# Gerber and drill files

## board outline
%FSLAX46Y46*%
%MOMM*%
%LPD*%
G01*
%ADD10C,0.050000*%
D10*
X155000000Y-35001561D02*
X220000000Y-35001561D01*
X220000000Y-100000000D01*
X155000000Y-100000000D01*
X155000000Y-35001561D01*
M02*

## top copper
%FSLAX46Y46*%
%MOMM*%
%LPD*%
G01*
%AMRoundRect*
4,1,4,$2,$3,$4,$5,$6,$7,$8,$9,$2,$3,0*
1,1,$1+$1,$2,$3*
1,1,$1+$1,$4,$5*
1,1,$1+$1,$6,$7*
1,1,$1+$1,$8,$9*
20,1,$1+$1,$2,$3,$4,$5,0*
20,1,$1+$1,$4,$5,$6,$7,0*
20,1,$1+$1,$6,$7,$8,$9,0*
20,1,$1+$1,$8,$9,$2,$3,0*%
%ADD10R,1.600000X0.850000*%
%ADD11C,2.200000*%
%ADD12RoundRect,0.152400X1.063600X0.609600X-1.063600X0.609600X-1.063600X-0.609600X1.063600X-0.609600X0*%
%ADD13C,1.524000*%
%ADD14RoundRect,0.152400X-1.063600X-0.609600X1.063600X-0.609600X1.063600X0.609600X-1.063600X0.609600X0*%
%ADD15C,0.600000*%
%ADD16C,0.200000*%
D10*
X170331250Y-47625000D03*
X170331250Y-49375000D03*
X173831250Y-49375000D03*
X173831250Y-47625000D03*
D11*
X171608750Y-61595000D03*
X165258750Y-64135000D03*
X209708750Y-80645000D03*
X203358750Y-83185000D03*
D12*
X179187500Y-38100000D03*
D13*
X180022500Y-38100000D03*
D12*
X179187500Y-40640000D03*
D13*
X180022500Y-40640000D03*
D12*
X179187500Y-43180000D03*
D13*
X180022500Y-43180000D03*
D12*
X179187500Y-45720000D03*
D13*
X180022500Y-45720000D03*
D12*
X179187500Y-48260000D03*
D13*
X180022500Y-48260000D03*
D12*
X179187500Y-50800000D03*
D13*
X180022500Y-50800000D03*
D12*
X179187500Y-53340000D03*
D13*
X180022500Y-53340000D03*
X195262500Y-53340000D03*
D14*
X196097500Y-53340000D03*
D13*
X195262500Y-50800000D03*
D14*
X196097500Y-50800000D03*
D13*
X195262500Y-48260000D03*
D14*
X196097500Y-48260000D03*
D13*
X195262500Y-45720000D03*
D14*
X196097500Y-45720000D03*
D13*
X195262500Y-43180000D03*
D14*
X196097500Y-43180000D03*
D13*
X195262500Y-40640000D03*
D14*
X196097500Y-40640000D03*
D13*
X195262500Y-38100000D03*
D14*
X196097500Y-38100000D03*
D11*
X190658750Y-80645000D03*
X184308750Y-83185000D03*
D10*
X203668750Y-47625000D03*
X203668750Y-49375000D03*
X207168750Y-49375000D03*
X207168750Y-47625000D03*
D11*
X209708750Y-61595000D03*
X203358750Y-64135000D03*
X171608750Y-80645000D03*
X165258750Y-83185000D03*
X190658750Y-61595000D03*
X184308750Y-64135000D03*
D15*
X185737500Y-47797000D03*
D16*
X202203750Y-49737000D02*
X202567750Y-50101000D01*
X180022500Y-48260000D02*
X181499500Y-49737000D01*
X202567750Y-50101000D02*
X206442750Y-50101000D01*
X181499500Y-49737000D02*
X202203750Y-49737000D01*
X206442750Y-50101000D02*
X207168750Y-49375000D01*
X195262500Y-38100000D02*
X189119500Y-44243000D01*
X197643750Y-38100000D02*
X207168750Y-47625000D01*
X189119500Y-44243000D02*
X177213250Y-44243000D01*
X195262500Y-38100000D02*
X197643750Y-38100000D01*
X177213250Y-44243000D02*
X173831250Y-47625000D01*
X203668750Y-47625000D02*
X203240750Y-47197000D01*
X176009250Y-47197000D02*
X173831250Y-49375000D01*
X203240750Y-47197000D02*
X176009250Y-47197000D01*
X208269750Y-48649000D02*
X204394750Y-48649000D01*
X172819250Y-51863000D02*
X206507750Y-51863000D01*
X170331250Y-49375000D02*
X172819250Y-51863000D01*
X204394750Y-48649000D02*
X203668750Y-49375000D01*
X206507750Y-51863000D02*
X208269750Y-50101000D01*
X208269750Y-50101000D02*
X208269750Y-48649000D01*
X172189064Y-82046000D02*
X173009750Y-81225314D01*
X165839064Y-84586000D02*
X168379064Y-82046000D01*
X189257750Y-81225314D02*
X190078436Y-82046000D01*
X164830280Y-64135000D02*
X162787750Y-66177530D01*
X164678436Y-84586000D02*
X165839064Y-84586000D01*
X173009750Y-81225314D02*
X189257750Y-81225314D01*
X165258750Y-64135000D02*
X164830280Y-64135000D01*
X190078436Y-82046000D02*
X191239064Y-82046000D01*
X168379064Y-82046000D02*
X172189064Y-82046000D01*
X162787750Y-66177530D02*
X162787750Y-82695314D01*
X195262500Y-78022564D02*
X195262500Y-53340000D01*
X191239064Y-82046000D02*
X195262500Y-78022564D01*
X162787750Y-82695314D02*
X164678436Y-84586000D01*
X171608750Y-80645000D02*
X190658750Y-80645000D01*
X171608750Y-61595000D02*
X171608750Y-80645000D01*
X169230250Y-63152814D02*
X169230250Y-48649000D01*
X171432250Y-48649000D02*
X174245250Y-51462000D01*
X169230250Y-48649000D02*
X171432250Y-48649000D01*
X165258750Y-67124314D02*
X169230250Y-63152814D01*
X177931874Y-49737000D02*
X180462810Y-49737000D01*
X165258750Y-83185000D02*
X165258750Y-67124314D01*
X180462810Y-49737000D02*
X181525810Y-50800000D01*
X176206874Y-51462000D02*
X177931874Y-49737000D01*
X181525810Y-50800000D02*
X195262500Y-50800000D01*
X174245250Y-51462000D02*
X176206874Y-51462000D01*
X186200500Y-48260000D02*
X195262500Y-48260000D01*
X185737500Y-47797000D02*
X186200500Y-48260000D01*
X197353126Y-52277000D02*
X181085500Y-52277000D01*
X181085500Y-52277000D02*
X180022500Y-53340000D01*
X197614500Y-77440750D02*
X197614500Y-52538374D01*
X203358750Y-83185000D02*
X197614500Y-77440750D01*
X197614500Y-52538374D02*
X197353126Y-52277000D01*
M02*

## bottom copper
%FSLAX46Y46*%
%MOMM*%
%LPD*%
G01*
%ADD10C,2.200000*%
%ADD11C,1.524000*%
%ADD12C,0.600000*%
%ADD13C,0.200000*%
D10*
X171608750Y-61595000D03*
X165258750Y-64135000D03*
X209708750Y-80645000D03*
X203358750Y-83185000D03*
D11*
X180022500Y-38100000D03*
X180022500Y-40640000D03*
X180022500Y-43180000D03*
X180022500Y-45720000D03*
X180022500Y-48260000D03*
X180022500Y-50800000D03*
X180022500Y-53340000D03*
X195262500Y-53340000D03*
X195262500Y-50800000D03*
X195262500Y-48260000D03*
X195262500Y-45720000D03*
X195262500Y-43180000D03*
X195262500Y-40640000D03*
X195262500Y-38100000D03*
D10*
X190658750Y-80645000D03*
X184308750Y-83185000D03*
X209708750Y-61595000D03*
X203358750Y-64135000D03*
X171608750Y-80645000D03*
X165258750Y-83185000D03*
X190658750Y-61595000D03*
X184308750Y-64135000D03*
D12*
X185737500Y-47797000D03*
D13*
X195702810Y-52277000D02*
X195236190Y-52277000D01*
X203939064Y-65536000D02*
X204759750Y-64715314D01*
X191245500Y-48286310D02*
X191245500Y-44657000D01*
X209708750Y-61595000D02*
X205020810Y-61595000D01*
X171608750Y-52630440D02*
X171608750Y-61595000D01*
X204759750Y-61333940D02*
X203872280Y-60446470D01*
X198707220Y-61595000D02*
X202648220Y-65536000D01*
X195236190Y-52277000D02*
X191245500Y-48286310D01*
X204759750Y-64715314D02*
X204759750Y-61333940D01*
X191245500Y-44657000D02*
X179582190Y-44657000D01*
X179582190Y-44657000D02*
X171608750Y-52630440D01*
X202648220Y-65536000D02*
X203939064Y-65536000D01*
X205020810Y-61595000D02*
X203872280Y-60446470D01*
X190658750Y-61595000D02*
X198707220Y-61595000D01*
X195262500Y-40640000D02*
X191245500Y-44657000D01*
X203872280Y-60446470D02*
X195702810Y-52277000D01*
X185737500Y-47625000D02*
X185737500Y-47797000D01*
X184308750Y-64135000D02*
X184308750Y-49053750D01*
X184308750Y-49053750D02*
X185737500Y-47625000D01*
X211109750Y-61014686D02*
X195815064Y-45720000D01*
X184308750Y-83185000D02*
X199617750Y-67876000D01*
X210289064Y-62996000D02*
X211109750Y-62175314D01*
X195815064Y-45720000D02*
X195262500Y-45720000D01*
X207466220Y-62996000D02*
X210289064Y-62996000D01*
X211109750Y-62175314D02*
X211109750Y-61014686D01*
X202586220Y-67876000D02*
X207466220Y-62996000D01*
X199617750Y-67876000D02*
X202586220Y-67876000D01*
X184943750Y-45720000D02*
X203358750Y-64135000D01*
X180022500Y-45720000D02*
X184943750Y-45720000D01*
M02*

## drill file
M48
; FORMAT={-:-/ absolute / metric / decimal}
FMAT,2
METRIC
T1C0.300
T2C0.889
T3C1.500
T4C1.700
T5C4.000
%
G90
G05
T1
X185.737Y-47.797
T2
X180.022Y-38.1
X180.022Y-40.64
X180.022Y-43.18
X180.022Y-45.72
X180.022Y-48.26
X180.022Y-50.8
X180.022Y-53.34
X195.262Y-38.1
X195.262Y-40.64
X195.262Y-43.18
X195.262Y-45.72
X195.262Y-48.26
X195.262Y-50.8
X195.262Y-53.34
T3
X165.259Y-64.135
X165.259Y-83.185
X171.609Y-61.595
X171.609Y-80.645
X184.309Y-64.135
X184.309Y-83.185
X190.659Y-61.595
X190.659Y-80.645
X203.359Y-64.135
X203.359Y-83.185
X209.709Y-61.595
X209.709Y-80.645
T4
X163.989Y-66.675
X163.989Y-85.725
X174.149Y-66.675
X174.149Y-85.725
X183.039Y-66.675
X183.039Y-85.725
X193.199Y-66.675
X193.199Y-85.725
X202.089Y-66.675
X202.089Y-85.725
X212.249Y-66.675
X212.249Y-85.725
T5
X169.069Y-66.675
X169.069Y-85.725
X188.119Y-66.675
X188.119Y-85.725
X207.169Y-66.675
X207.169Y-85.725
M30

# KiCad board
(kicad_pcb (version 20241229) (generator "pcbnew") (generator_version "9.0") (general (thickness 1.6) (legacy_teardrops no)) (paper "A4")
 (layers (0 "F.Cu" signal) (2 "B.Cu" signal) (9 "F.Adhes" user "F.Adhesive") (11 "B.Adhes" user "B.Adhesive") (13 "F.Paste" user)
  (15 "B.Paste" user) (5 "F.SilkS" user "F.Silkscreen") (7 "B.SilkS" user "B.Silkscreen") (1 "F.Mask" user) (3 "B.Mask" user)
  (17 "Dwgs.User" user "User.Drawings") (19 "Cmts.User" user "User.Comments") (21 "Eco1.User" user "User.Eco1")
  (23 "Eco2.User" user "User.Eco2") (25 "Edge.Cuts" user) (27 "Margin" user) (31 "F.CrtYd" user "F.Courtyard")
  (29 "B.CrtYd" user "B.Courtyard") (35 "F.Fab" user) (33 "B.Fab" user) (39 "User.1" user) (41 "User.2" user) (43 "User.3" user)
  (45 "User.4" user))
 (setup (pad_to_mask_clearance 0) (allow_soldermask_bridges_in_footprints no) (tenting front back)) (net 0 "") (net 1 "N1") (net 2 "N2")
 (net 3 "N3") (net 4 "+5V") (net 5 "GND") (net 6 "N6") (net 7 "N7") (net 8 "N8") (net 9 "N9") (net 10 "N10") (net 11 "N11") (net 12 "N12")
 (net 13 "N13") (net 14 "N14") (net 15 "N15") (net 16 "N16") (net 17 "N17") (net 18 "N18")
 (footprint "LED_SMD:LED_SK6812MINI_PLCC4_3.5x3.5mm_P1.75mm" (layer "F.Cu") (at 172.08125 48.5)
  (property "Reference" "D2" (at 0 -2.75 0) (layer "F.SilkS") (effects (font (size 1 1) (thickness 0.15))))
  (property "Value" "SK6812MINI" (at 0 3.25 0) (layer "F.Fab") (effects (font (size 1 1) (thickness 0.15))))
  (pad "1" smd rect (at -1.75 -0.875) (size 1.6 0.85) (layers "F.Cu" "F.Mask" "F.Paste") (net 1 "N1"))
  (pad "2" smd rect (at -1.75 0.875) (size 1.6 0.85) (layers "F.Cu" "F.Mask" "F.Paste") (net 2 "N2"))
  (pad "3" smd rect (at 1.75 0.875) (size 1.6 0.85) (layers "F.Cu" "F.Mask" "F.Paste") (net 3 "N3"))
  (pad "4" smd rect (at 1.75 -0.875) (size 1.6 0.85) (layers "F.Cu" "F.Mask" "F.Paste") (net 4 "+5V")))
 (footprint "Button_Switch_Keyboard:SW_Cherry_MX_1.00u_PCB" (layer "F.Cu") (at 171.60875 61.595)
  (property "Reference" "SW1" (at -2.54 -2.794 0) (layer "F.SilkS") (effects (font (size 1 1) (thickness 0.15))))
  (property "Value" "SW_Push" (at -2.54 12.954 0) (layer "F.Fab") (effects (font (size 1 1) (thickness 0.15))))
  (pad "" np_thru_hole circle (at -7.62 5.08) (size 1.7 1.7) (drill 1.7) (layers "*.Cu" "*.Mask"))
  (pad "" np_thru_hole circle (at -2.54 5.08) (size 4 4) (drill 4) (layers "*.Cu" "*.Mask"))
  (pad "" np_thru_hole circle (at 2.54 5.08) (size 1.7 1.7) (drill 1.7) (layers "*.Cu" "*.Mask"))
  (pad "1" thru_hole circle (at 0 0) (size 2.2 2.2) (drill 1.5) (layers "*.Cu" "*.Mask") (remove_unused_layers no) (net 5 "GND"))
  (pad "2" thru_hole circle (at -6.35 2.54) (size 2.2 2.2) (drill 1.5) (layers "*.Cu" "*.Mask") (remove_unused_layers no) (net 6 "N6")))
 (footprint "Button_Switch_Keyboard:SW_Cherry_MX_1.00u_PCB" (layer "F.Cu") (at 209.70875 80.645)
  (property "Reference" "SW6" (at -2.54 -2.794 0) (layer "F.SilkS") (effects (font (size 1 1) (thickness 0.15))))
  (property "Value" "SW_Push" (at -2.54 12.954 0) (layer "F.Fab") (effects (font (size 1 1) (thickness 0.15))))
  (pad "" np_thru_hole circle (at -7.62 5.08) (size 1.7 1.7) (drill 1.7) (layers "*.Cu" "*.Mask"))
  (pad "" np_thru_hole circle (at -2.54 5.08) (size 4 4) (drill 4) (layers "*.Cu" "*.Mask"))
  (pad "" np_thru_hole circle (at 2.54 5.08) (size 1.7 1.7) (drill 1.7) (layers "*.Cu" "*.Mask"))
  (pad "1" thru_hole circle (at 0 0) (size 2.2 2.2) (drill 1.5) (layers "*.Cu" "*.Mask") (remove_unused_layers no) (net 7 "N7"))
  (pad "2" thru_hole circle (at -6.35 2.54) (size 2.2 2.2) (drill 1.5) (layers "*.Cu" "*.Mask") (remove_unused_layers no) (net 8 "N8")))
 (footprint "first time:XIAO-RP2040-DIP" (layer "F.Cu") (at 187.6425 45.72)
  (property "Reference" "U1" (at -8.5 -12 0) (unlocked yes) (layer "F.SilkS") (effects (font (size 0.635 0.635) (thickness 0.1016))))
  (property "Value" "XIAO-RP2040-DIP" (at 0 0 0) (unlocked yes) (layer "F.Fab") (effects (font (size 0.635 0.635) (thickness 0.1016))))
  (pad "1" smd roundrect (at -8.455 -7.62 180) (size 2.432 1.524) (layers "F.Cu" "F.Mask") (roundrect_rratio 0.1) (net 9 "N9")
   (thermal_bridge_angle 45))
  (pad "1" thru_hole circle (at -7.62 -7.62 180) (size 1.524 1.524) (drill 0.889) (layers "*.Cu" "*.Mask") (remove_unused_layers no)
   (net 9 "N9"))
  (pad "2" smd roundrect (at -8.455 -5.08 180) (size 2.432 1.524) (layers "F.Cu" "F.Mask") (roundrect_rratio 0.1) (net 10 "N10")
   (thermal_bridge_angle 45))
  (pad "2" thru_hole circle (at -7.62 -5.08 180) (size 1.524 1.524) (drill 0.889) (layers "*.Cu" "*.Mask") (remove_unused_layers no)
   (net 10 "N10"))
  (pad "3" smd roundrect (at -8.455 -2.54 180) (size 2.432 1.524) (layers "F.Cu" "F.Mask") (roundrect_rratio 0.1) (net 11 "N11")
   (thermal_bridge_angle 45))
  (pad "3" thru_hole circle (at -7.62 -2.54 180) (size 1.524 1.524) (drill 0.889) (layers "*.Cu" "*.Mask") (remove_unused_layers no)
   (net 11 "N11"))
  (pad "4" smd roundrect (at -8.455 0 180) (size 2.432 1.524) (layers "F.Cu" "F.Mask") (roundrect_rratio 0.1) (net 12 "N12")
   (thermal_bridge_angle 45))
  (pad "4" thru_hole circle (at -7.62 0 180) (size 1.524 1.524) (drill 0.889) (layers "*.Cu" "*.Mask") (remove_unused_layers no)
   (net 12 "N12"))
  (pad "5" smd roundrect (at -8.455 2.54 180) (size 2.432 1.524) (layers "F.Cu" "F.Mask") (roundrect_rratio 0.1) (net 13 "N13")
   (thermal_bridge_angle 45))
  (pad "5" thru_hole circle (at -7.62 2.54 180) (size 1.524 1.524) (drill 0.889) (layers "*.Cu" "*.Mask") (remove_unused_layers no)
   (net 13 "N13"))
  (pad "6" smd roundrect (at -8.455 5.08 180) (size 2.432 1.524) (layers "F.Cu" "F.Mask") (roundrect_rratio 0.1) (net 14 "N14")
   (thermal_bridge_angle 45))
  (pad "6" thru_hole circle (at -7.62 5.08 180) (size 1.524 1.524) (drill 0.889) (layers "*.Cu" "*.Mask") (remove_unused_layers no)
   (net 14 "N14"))
  (pad "7" smd roundrect (at -8.455 7.62 180) (size 2.432 1.524) (layers "F.Cu" "F.Mask") (roundrect_rratio 0.1) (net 8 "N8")
   (thermal_bridge_angle 45))
  (pad "7" thru_hole circle (at -7.62 7.62 180) (size 1.524 1.524) (drill 0.889) (layers "*.Cu" "*.Mask") (remove_unused_layers no)
   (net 8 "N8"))
  (pad "8" thru_hole circle (at 7.62 7.62) (size 1.524 1.524) (drill 0.889) (layers "*.Cu" "*.Mask") (remove_unused_layers no) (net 6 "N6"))
  (pad "8" smd roundrect (at 8.455 7.62) (size 2.432 1.524) (layers "F.Cu" "F.Mask") (roundrect_rratio 0.1) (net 6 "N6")
   (thermal_bridge_angle 45))
  (pad "9" thru_hole circle (at 7.62 5.08) (size 1.524 1.524) (drill 0.889) (layers "*.Cu" "*.Mask") (remove_unused_layers no)
   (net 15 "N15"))
  (pad "9" smd roundrect (at 8.455 5.08) (size 2.432 1.524) (layers "F.Cu" "F.Mask") (roundrect_rratio 0.1) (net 15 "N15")
   (thermal_bridge_angle 45))
  (pad "10" thru_hole circle (at 7.62 2.54) (size 1.524 1.524) (drill 0.889) (layers "*.Cu" "*.Mask") (remove_unused_layers no)
   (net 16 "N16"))
  (pad "10" smd roundrect (at 8.455 2.54) (size 2.432 1.524) (layers "F.Cu" "F.Mask") (roundrect_rratio 0.1) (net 16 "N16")
   (thermal_bridge_angle 45))
  (pad "11" thru_hole circle (at 7.62 0) (size 1.524 1.524) (drill 0.889) (layers "*.Cu" "*.Mask") (remove_unused_layers no) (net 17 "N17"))
  (pad "11" smd roundrect (at 8.455 0) (size 2.432 1.524) (layers "F.Cu" "F.Mask") (roundrect_rratio 0.1) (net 17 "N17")
   (thermal_bridge_angle 45))
  (pad "12" thru_hole circle (at 7.62 -2.54) (size 1.524 1.524) (drill 0.889) (layers "*.Cu" "*.Mask") (remove_unused_layers no)
   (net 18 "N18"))
  (pad "12" smd roundrect (at 8.455 -2.54) (size 2.432 1.524) (layers "F.Cu" "F.Mask") (roundrect_rratio 0.1) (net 18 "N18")
   (thermal_bridge_angle 45))
  (pad "13" thru_hole circle (at 7.62 -5.08) (size 1.524 1.524) (drill 0.889) (layers "*.Cu" "*.Mask") (remove_unused_layers no)
   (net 5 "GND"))
  (pad "13" smd roundrect (at 8.455 -5.08) (size 2.432 1.524) (layers "F.Cu" "F.Mask") (roundrect_rratio 0.1) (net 5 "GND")
   (thermal_bridge_angle 45))
  (pad "14" thru_hole circle (at 7.62 -7.62) (size 1.524 1.524) (drill 0.889) (layers "*.Cu" "*.Mask") (remove_unused_layers no)
   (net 4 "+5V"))
  (pad "14" smd roundrect (at 8.455 -7.62) (size 2.432 1.524) (layers "F.Cu" "F.Mask") (roundrect_rratio 0.1) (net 4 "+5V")
   (thermal_bridge_angle 45)))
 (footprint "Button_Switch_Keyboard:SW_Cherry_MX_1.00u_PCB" (layer "F.Cu") (at 190.65875 80.645)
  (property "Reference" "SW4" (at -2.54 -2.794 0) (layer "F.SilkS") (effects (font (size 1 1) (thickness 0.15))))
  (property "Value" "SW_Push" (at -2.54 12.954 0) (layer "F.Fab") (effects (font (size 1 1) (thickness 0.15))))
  (pad "" np_thru_hole circle (at -7.62 5.08) (size 1.7 1.7) (drill 1.7) (layers "*.Cu" "*.Mask"))
  (pad "" np_thru_hole circle (at -2.54 5.08) (size 4 4) (drill 4) (layers "*.Cu" "*.Mask"))
  (pad "" np_thru_hole circle (at 2.54 5.08) (size 1.7 1.7) (drill 1.7) (layers "*.Cu" "*.Mask"))
  (pad "1" thru_hole circle (at 0 0) (size 2.2 2.2) (drill 1.5) (layers "*.Cu" "*.Mask") (remove_unused_layers no) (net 5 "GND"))
  (pad "2" thru_hole circle (at -6.35 2.54) (size 2.2 2.2) (drill 1.5) (layers "*.Cu" "*.Mask") (remove_unused_layers no) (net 17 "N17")))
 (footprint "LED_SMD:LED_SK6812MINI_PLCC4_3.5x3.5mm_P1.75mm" (layer "F.Cu") (at 205.41875 48.5)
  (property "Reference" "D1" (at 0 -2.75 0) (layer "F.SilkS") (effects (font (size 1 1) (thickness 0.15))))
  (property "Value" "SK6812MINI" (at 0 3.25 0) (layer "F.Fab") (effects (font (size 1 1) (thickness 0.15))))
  (pad "1" smd rect (at -1.75 -0.875) (size 1.6 0.85) (layers "F.Cu" "F.Mask" "F.Paste") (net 3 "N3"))
  (pad "2" smd rect (at -1.75 0.875) (size 1.6 0.85) (layers "F.Cu" "F.Mask" "F.Paste") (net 2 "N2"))
  (pad "3" smd rect (at 1.75 0.875) (size 1.6 0.85) (layers "F.Cu" "F.Mask" "F.Paste") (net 13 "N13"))
  (pad "4" smd rect (at 1.75 -0.875) (size 1.6 0.85) (layers "F.Cu" "F.Mask" "F.Paste") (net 4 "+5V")))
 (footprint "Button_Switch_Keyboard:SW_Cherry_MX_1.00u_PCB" (layer "F.Cu") (at 209.70875 61.595)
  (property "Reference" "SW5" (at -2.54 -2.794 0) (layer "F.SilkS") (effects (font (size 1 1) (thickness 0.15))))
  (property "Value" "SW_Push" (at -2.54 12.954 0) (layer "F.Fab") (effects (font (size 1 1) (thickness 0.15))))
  (pad "" np_thru_hole circle (at -7.62 5.08) (size 1.7 1.7) (drill 1.7) (layers "*.Cu" "*.Mask"))
  (pad "" np_thru_hole circle (at -2.54 5.08) (size 4 4) (drill 4) (layers "*.Cu" "*.Mask"))
  (pad "" np_thru_hole circle (at 2.54 5.08) (size 1.7 1.7) (drill 1.7) (layers "*.Cu" "*.Mask"))
  (pad "1" thru_hole circle (at 0 0) (size 2.2 2.2) (drill 1.5) (layers "*.Cu" "*.Mask") (remove_unused_layers no) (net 5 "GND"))
  (pad "2" thru_hole circle (at -6.35 2.54) (size 2.2 2.2) (drill 1.5) (layers "*.Cu" "*.Mask") (remove_unused_layers no) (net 12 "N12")))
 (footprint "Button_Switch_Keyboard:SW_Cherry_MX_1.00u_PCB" (layer "F.Cu") (at 171.60875 80.645)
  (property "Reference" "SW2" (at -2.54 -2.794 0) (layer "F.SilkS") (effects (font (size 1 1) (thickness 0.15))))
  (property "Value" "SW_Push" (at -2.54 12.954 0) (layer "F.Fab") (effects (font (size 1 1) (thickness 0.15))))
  (pad "" np_thru_hole circle (at -7.62 5.08) (size 1.7 1.7) (drill 1.7) (layers "*.Cu" "*.Mask"))
  (pad "" np_thru_hole circle (at -2.54 5.08) (size 4 4) (drill 4) (layers "*.Cu" "*.Mask"))
  (pad "" np_thru_hole circle (at 2.54 5.08) (size 1.7 1.7) (drill 1.7) (layers "*.Cu" "*.Mask"))
  (pad "1" thru_hole circle (at 0 0) (size 2.2 2.2) (drill 1.5) (layers "*.Cu" "*.Mask") (remove_unused_layers no) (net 5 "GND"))
  (pad "2" thru_hole circle (at -6.35 2.54) (size 2.2 2.2) (drill 1.5) (layers "*.Cu" "*.Mask") (remove_unused_layers no) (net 15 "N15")))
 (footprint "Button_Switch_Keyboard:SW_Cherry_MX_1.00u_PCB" (layer "F.Cu") (at 190.65875 61.595)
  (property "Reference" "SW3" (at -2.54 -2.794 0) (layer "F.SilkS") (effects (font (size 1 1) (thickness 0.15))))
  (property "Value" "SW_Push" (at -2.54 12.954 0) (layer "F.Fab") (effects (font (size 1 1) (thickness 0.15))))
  (pad "" np_thru_hole circle (at -7.62 5.08) (size 1.7 1.7) (drill 1.7) (layers "*.Cu" "*.Mask"))
  (pad "" np_thru_hole circle (at -2.54 5.08) (size 4 4) (drill 4) (layers "*.Cu" "*.Mask"))
  (pad "" np_thru_hole circle (at 2.54 5.08) (size 1.7 1.7) (drill 1.7) (layers "*.Cu" "*.Mask"))
  (pad "1" thru_hole circle (at 0 0) (size 2.2 2.2) (drill 1.5) (layers "*.Cu" "*.Mask") (remove_unused_layers no) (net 5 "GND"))
  (pad "2" thru_hole circle (at -6.35 2.54) (size 2.2 2.2) (drill 1.5) (layers "*.Cu" "*.Mask") (remove_unused_layers no) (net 16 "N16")))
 (gr_rect (start 155 35.001561) (end 220 100) (stroke (width 0.05) (type default)) (fill no) (layer "Edge.Cuts"))
 (segment (start 202.20375 49.737) (end 202.56775 50.101) (width 0.2) (layer "F.Cu") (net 13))
 (segment (start 180.0225 48.26) (end 181.4995 49.737) (width 0.2) (layer "F.Cu") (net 13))
 (segment (start 202.56775 50.101) (end 206.44275 50.101) (width 0.2) (layer "F.Cu") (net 13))
 (segment (start 181.4995 49.737) (end 202.20375 49.737) (width 0.2) (layer "F.Cu") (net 13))
 (segment (start 206.44275 50.101) (end 207.16875 49.375) (width 0.2) (layer "F.Cu") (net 13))
 (segment (start 195.2625 38.1) (end 189.1195 44.243) (width 0.2) (layer "F.Cu") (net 4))
 (segment (start 197.64375 38.1) (end 207.16875 47.625) (width 0.2) (layer "F.Cu") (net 4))
 (segment (start 189.1195 44.243) (end 177.21325 44.243) (width 0.2) (layer "F.Cu") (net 4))
 (segment (start 195.2625 38.1) (end 197.64375 38.1) (width 0.2) (layer "F.Cu") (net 4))
 (segment (start 177.21325 44.243) (end 173.83125 47.625) (width 0.2) (layer "F.Cu") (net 4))
 (segment (start 203.66875 47.625) (end 203.24075 47.197) (width 0.2) (layer "F.Cu") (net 3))
 (segment (start 176.00925 47.197) (end 173.83125 49.375) (width 0.2) (layer "F.Cu") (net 3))
 (segment (start 203.24075 47.197) (end 176.00925 47.197) (width 0.2) (layer "F.Cu") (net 3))
 (segment (start 208.26975 48.649) (end 204.39475 48.649) (width 0.2) (layer "F.Cu") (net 2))
 (segment (start 172.81925 51.863) (end 206.50775 51.863) (width 0.2) (layer "F.Cu") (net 2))
 (segment (start 170.33125 49.375) (end 172.81925 51.863) (width 0.2) (layer "F.Cu") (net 2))
 (segment (start 204.39475 48.649) (end 203.66875 49.375) (width 0.2) (layer "F.Cu") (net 2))
 (segment (start 206.50775 51.863) (end 208.26975 50.101) (width 0.2) (layer "F.Cu") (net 2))
 (segment (start 208.26975 50.101) (end 208.26975 48.649) (width 0.2) (layer "F.Cu") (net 2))
 (segment (start 172.189064 82.046) (end 173.00975 81.225314) (width 0.2) (layer "F.Cu") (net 6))
 (segment (start 165.839064 84.586) (end 168.379064 82.046) (width 0.2) (layer "F.Cu") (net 6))
 (segment (start 189.25775 81.225314) (end 190.078436 82.046) (width 0.2) (layer "F.Cu") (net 6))
 (segment (start 164.83028 64.135) (end 162.78775 66.17753) (width 0.2) (layer "F.Cu") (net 6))
 (segment (start 164.678436 84.586) (end 165.839064 84.586) (width 0.2) (layer "F.Cu") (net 6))
 (segment (start 173.00975 81.225314) (end 189.25775 81.225314) (width 0.2) (layer "F.Cu") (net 6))
 (segment (start 165.25875 64.135) (end 164.83028 64.135) (width 0.2) (layer "F.Cu") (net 6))
 (segment (start 190.078436 82.046) (end 191.239064 82.046) (width 0.2) (layer "F.Cu") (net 6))
 (segment (start 168.379064 82.046) (end 172.189064 82.046) (width 0.2) (layer "F.Cu") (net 6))
 (segment (start 162.78775 66.17753) (end 162.78775 82.695314) (width 0.2) (layer "F.Cu") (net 6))
 (segment (start 195.2625 78.022564) (end 195.2625 53.34) (width 0.2) (layer "F.Cu") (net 6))
 (segment (start 191.239064 82.046) (end 195.2625 78.022564) (width 0.2) (layer "F.Cu") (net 6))
 (segment (start 162.78775 82.695314) (end 164.678436 84.586) (width 0.2) (layer "F.Cu") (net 6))
 (segment (start 171.60875 80.645) (end 190.65875 80.645) (width 0.2) (layer "F.Cu") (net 5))
 (segment (start 171.60875 61.595) (end 171.60875 80.645) (width 0.2) (layer "F.Cu") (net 5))
 (segment (start 195.70281 52.277) (end 195.23619 52.277) (width 0.2) (layer "B.Cu") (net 5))
 (segment (start 203.939064 65.536) (end 204.75975 64.715314) (width 0.2) (layer "B.Cu") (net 5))
 (segment (start 191.2455 48.28631) (end 191.2455 44.657) (width 0.2) (layer "B.Cu") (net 5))
 (segment (start 209.70875 61.595) (end 205.02081 61.595) (width 0.2) (layer "B.Cu") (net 5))
 (segment (start 171.60875 52.63044) (end 171.60875 61.595) (width 0.2) (layer "B.Cu") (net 5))
 (segment (start 204.75975 61.33394) (end 203.87228 60.44647) (width 0.2) (layer "B.Cu") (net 5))
 (segment (start 198.70722 61.595) (end 202.64822 65.536) (width 0.2) (layer "B.Cu") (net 5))
 (segment (start 195.23619 52.277) (end 191.2455 48.28631) (width 0.2) (layer "B.Cu") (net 5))
 (segment (start 204.75975 64.715314) (end 204.75975 61.33394) (width 0.2) (layer "B.Cu") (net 5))
 (segment (start 191.2455 44.657) (end 179.58219 44.657) (width 0.2) (layer "B.Cu") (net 5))
 (segment (start 179.58219 44.657) (end 171.60875 52.63044) (width 0.2) (layer "B.Cu") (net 5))
 (segment (start 202.64822 65.536) (end 203.939064 65.536) (width 0.2) (layer "B.Cu") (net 5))
 (segment (start 205.02081 61.595) (end 203.87228 60.44647) (width 0.2) (layer "B.Cu") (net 5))
 (segment (start 190.65875 61.595) (end 198.70722 61.595) (width 0.2) (layer "B.Cu") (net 5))
 (segment (start 195.2625 40.64) (end 191.2455 44.657) (width 0.2) (layer "B.Cu") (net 5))
 (segment (start 203.87228 60.44647) (end 195.70281 52.277) (width 0.2) (layer "B.Cu") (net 5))
 (segment (start 169.23025 63.152814) (end 169.23025 48.649) (width 0.2) (layer "F.Cu") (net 15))
 (segment (start 171.43225 48.649) (end 174.24525 51.462) (width 0.2) (layer "F.Cu") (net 15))
 (segment (start 169.23025 48.649) (end 171.43225 48.649) (width 0.2) (layer "F.Cu") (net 15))
 (segment (start 165.25875 67.124314) (end 169.23025 63.152814) (width 0.2) (layer "F.Cu") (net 15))
 (segment (start 177.931874 49.737) (end 180.46281 49.737) (width 0.2) (layer "F.Cu") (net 15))
 (segment (start 165.25875 83.185) (end 165.25875 67.124314) (width 0.2) (layer "F.Cu") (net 15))
 (segment (start 180.46281 49.737) (end 181.52581 50.8) (width 0.2) (layer "F.Cu") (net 15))
 (segment (start 176.206874 51.462) (end 177.931874 49.737) (width 0.2) (layer "F.Cu") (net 15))
 (segment (start 181.52581 50.8) (end 195.2625 50.8) (width 0.2) (layer "F.Cu") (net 15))
 (segment (start 174.24525 51.462) (end 176.206874 51.462) (width 0.2) (layer "F.Cu") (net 15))
 (segment (start 186.2005 48.26) (end 195.2625 48.26) (width 0.2) (layer "F.Cu") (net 16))
 (segment (start 185.7375 47.797) (end 186.2005 48.26) (width 0.2) (layer "F.Cu") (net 16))
 (via (at 185.7375 47.797) (size 0.6) (drill 0.3) (layers "F.Cu" "B.Cu") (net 16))
 (segment (start 185.7375 47.625) (end 185.7375 47.797) (width 0.2) (layer "B.Cu") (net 16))
 (segment (start 184.30875 64.135) (end 184.30875 49.05375) (width 0.2) (layer "B.Cu") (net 16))
 (segment (start 184.30875 49.05375) (end 185.7375 47.625) (width 0.2) (layer "B.Cu") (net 16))
 (segment (start 211.10975 61.014686) (end 195.815064 45.72) (width 0.2) (layer "B.Cu") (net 17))
 (segment (start 184.30875 83.185) (end 199.61775 67.876) (width 0.2) (layer "B.Cu") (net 17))
 (segment (start 210.289064 62.996) (end 211.10975 62.175314) (width 0.2) (layer "B.Cu") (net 17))
 (segment (start 195.815064 45.72) (end 195.2625 45.72) (width 0.2) (layer "B.Cu") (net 17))
 (segment (start 207.46622 62.996) (end 210.289064 62.996) (width 0.2) (layer "B.Cu") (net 17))
 (segment (start 211.10975 62.175314) (end 211.10975 61.014686) (width 0.2) (layer "B.Cu") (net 17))
 (segment (start 202.58622 67.876) (end 207.46622 62.996) (width 0.2) (layer "B.Cu") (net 17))
 (segment (start 199.61775 67.876) (end 202.58622 67.876) (width 0.2) (layer "B.Cu") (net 17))
 (segment (start 184.94375 45.72) (end 203.35875 64.135) (width 0.2) (layer "B.Cu") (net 12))
 (segment (start 180.0225 45.72) (end 184.94375 45.72) (width 0.2) (layer "B.Cu") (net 12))
 (segment (start 197.353126 52.277) (end 181.0855 52.277) (width 0.2) (layer "F.Cu") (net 8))
 (segment (start 181.0855 52.277) (end 180.0225 53.34) (width 0.2) (layer "F.Cu") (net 8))
 (segment (start 197.6145 77.44075) (end 197.6145 52.538374) (width 0.2) (layer "F.Cu") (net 8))
 (segment (start 203.35875 83.185) (end 197.6145 77.44075) (width 0.2) (layer "F.Cu") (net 8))
 (segment (start 197.6145 52.538374) (end 197.353126 52.277) (width 0.2) (layer "F.Cu") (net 8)))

